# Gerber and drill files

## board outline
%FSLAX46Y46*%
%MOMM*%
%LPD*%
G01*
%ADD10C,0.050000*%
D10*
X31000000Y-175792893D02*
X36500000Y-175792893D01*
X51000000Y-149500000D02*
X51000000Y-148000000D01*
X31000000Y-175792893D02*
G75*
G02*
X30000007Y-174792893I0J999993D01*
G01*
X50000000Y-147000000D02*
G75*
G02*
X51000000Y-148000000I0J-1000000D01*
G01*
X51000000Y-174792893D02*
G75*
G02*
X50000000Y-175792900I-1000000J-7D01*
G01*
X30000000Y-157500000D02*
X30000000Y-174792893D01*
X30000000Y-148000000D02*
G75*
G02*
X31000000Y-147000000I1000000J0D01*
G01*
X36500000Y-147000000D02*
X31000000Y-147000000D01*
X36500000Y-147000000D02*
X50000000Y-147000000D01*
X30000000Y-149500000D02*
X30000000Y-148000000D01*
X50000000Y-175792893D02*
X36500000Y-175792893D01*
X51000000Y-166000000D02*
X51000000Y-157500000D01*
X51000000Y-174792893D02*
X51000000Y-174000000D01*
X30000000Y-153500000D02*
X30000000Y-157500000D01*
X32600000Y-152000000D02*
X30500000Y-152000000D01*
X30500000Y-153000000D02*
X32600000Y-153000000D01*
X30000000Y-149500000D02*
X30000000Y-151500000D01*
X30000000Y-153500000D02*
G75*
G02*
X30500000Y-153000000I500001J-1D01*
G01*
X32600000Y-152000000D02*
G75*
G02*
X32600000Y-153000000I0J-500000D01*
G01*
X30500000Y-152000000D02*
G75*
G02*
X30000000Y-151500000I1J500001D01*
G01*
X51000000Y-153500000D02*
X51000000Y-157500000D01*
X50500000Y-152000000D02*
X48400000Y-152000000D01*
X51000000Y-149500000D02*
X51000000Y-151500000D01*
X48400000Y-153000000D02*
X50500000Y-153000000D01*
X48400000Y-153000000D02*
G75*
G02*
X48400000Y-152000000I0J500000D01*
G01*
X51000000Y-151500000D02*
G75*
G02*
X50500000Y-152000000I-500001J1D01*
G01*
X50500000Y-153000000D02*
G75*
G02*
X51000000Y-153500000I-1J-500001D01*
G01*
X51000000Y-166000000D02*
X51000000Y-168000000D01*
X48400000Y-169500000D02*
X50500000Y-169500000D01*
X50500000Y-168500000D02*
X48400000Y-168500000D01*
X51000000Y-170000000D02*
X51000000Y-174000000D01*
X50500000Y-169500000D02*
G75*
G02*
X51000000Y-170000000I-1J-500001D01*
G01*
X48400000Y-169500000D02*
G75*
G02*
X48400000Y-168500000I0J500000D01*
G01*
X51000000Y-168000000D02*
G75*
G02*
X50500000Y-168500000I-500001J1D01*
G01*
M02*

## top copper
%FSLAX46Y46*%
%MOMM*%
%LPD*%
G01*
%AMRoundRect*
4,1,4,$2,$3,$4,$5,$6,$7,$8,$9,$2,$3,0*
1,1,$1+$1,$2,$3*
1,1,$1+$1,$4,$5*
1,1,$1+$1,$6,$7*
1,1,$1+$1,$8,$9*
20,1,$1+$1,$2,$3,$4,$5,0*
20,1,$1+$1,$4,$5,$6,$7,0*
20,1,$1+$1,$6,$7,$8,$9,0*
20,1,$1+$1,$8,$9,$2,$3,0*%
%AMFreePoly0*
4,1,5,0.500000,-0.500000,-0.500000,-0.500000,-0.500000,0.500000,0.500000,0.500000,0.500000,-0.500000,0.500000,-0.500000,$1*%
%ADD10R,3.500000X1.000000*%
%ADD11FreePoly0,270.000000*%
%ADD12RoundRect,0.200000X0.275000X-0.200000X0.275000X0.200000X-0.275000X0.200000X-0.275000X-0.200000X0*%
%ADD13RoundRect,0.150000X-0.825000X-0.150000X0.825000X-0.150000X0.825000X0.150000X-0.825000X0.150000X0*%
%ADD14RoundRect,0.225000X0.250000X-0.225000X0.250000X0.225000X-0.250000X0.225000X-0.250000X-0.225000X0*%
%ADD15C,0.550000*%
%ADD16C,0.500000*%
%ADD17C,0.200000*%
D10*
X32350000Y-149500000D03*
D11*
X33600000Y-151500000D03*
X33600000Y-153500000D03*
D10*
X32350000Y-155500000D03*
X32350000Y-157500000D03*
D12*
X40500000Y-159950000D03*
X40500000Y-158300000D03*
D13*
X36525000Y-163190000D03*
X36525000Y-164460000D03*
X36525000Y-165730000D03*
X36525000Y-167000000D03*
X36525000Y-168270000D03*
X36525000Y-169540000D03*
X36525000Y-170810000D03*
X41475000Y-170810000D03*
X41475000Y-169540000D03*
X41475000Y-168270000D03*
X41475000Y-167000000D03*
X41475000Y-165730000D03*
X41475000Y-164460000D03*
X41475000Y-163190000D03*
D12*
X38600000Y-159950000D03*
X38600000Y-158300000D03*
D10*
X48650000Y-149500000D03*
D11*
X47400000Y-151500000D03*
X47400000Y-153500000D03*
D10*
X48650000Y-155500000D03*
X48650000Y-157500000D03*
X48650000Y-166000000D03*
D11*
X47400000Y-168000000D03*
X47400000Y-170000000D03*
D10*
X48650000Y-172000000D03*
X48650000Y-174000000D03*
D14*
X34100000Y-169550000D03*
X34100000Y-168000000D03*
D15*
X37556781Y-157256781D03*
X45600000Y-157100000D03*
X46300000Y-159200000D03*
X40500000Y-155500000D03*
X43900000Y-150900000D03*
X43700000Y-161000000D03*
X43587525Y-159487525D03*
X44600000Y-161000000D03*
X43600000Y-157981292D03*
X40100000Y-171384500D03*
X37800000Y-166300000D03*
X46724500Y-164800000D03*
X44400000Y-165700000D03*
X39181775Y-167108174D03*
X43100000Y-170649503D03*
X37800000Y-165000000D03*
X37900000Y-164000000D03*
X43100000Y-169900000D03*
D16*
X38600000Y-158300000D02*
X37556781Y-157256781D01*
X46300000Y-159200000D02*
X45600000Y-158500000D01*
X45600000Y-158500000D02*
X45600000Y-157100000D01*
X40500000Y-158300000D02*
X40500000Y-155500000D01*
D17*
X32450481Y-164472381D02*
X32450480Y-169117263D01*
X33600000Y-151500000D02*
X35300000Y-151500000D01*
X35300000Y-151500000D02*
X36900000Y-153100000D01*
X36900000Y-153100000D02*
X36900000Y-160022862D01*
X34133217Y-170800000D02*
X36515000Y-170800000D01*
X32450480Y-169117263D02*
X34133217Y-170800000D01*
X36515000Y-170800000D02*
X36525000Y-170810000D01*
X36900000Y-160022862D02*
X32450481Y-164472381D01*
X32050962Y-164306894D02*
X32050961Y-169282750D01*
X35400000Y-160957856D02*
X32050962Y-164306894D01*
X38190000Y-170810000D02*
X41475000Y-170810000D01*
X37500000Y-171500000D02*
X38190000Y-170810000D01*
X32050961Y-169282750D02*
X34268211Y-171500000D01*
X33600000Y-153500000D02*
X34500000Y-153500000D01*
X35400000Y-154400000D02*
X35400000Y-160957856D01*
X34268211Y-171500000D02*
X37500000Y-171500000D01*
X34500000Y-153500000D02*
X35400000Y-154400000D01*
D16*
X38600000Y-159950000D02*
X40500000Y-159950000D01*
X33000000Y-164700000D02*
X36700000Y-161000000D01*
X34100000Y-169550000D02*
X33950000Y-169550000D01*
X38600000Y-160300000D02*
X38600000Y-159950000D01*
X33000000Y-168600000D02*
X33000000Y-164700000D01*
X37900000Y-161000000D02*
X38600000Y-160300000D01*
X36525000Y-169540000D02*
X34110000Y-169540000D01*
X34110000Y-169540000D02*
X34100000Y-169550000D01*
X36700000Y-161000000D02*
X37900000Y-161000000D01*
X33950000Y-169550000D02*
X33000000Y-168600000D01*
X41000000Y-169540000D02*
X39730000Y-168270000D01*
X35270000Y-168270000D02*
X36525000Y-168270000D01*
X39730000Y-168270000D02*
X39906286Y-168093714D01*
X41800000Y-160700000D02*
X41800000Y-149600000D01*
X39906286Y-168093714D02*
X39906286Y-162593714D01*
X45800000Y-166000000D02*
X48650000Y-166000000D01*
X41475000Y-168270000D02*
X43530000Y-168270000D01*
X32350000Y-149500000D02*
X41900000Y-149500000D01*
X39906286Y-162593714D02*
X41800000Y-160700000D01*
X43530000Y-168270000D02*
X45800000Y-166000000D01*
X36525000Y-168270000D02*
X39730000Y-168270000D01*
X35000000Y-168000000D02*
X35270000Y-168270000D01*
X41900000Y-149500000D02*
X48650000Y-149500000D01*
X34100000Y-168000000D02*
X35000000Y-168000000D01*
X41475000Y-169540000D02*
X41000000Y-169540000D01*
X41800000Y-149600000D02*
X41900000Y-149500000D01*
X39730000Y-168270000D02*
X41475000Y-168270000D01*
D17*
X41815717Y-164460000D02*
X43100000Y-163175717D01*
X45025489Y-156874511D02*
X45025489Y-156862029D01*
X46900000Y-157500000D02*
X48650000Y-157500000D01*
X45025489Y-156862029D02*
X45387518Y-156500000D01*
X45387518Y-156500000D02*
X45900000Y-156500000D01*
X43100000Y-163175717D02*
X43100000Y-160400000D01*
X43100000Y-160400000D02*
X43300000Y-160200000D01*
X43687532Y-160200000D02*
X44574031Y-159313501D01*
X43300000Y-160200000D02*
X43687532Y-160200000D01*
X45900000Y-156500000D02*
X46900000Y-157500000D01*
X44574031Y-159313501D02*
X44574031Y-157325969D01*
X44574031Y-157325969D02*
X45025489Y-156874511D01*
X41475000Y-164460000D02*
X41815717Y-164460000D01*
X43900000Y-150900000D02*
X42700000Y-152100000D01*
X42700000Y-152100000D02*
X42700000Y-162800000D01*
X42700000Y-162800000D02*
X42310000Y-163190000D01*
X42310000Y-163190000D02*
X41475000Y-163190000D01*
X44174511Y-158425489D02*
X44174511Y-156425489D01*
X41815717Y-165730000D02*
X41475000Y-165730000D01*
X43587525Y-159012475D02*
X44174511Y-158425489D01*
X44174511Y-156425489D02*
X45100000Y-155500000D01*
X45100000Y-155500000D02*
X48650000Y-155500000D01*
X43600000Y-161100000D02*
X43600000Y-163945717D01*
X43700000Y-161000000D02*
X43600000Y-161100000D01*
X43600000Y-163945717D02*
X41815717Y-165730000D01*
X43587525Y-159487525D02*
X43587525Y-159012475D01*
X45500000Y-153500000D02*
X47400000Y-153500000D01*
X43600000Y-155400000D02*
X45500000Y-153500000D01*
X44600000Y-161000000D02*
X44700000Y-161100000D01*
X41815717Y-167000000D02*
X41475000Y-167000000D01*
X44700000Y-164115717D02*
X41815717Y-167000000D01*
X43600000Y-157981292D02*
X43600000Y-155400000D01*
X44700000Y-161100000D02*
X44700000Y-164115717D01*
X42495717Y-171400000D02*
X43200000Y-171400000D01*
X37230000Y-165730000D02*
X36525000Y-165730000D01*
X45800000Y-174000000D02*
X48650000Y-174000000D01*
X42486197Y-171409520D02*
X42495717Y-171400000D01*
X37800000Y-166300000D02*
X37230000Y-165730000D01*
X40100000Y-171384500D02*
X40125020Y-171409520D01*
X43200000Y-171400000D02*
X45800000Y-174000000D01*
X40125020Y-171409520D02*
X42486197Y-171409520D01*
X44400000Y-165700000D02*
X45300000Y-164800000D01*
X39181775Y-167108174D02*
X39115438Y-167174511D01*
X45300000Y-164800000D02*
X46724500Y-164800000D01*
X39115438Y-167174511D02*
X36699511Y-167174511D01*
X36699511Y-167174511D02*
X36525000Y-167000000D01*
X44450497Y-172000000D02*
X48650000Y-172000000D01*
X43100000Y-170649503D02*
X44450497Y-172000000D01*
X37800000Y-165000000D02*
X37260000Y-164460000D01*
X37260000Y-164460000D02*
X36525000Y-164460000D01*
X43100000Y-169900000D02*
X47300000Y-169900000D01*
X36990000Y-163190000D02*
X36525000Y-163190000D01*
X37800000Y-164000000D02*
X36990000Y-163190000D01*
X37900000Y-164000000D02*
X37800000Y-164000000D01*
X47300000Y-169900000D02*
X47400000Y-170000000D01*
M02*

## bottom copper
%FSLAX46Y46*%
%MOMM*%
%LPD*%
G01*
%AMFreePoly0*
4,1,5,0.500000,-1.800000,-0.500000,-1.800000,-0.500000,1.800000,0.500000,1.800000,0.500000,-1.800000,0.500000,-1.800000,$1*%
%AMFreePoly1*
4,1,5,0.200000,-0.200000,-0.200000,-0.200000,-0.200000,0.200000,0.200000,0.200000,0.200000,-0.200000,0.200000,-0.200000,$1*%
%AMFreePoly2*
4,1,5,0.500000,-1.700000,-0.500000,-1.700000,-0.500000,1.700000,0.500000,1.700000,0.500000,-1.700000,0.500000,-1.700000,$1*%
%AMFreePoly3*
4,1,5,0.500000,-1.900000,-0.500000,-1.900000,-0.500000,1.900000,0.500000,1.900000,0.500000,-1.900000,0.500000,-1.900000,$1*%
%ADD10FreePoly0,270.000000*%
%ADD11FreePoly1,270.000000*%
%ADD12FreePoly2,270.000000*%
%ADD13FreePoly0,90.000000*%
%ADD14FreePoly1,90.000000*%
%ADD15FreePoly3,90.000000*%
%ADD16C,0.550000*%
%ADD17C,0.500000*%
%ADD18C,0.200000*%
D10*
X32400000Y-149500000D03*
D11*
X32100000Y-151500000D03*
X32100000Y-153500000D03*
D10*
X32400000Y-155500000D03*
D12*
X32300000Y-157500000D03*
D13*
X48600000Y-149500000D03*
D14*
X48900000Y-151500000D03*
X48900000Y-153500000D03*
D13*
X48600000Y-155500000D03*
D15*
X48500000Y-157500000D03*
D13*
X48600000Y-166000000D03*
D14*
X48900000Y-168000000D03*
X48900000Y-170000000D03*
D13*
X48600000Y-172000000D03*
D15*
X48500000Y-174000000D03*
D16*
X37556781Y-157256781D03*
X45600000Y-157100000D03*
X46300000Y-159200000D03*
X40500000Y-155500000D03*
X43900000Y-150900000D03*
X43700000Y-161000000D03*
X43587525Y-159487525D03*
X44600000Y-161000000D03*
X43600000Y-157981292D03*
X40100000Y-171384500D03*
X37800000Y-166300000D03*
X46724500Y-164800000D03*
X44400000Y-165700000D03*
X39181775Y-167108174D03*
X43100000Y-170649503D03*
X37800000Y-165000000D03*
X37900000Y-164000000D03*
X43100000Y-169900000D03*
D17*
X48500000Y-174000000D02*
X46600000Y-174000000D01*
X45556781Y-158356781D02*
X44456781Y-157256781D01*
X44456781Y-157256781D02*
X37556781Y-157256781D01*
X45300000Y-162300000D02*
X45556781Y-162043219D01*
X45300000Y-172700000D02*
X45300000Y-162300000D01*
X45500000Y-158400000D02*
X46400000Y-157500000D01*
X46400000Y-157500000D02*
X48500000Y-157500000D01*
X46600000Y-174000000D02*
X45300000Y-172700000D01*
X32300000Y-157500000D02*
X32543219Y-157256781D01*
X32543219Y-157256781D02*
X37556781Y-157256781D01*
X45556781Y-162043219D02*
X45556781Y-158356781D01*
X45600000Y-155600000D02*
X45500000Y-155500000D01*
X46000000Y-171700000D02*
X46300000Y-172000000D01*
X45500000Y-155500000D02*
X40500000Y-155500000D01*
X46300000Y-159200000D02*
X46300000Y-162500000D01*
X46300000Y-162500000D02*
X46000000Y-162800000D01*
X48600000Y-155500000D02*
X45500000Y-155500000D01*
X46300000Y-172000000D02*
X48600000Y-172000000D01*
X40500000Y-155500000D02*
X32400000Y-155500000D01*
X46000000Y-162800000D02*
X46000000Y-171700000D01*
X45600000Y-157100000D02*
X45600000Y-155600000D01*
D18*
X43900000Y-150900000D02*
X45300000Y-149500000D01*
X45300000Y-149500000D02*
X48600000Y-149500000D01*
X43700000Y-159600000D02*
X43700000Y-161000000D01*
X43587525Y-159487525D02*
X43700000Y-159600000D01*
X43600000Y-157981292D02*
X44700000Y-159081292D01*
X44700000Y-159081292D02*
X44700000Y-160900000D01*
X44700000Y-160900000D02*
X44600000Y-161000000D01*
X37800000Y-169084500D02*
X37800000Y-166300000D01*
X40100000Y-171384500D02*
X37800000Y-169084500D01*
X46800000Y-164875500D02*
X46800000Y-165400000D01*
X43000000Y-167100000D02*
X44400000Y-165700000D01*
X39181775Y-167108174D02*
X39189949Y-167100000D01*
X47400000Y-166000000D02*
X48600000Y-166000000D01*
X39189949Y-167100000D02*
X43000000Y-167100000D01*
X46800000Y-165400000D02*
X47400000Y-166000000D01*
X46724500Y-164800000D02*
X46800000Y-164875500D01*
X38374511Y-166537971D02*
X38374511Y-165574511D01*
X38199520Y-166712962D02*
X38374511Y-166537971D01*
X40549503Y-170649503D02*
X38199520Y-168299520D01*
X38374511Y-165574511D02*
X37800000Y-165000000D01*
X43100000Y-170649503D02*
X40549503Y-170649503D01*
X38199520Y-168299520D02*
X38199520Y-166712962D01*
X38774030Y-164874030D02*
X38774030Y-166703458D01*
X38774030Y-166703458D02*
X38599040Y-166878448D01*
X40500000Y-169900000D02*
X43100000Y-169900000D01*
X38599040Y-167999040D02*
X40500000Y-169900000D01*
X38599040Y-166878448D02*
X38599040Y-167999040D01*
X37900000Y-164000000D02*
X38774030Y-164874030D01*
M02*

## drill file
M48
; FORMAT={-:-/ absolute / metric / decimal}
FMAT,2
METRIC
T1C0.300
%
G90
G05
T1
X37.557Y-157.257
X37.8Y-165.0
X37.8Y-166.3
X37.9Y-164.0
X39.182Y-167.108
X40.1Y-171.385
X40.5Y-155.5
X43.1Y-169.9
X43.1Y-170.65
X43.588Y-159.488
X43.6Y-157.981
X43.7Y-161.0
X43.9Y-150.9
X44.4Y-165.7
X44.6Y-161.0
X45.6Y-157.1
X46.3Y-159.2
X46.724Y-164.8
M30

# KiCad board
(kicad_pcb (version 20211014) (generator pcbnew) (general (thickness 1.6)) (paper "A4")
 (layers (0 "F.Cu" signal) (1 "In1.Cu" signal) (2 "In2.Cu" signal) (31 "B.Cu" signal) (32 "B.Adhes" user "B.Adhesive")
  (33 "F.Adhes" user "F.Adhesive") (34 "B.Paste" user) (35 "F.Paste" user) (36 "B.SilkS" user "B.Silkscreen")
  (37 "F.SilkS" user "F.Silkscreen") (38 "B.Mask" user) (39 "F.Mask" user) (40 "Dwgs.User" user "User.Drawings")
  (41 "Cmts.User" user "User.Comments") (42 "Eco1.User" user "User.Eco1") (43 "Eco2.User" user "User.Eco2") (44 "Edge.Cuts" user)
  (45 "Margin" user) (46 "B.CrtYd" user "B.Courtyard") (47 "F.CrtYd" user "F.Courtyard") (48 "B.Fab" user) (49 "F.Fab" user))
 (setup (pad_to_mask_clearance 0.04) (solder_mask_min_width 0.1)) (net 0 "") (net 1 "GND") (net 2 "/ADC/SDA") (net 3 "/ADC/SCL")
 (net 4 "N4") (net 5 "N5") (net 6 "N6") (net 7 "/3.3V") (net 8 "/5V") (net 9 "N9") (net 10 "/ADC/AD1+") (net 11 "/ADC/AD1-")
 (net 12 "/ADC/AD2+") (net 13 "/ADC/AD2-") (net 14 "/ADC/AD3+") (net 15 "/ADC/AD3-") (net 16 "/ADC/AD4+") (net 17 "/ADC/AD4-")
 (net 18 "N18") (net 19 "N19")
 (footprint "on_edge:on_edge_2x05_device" (layer "F.Cu") (at 30 153.5 -90)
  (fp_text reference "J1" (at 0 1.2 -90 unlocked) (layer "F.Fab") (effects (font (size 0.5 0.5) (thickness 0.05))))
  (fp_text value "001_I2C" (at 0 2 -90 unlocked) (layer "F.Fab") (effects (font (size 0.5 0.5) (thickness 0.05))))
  (fp_line (start 0 0) (end 4 0) (layer "Edge.Cuts") (width 0.05))
  (fp_line (start -1.5 -2.6) (end -1.5 -0.5) (layer "Edge.Cuts") (width 0.05))
  (fp_line (start -0.5 -0.5) (end -0.5 -2.6) (layer "Edge.Cuts") (width 0.05))
  (fp_line (start -4 0) (end -2 0) (layer "Edge.Cuts") (width 0.05))
  (fp_arc (start 0 0) (mid -0.353553 -0.146447) (end -0.5 -0.5) (layer "Edge.Cuts") (width 0.05))
  (fp_arc (start -1.5 -2.6) (mid -1 -3.1) (end -0.5 -2.6) (layer "Edge.Cuts") (width 0.05))
  (fp_arc (start -1.5 -0.5) (mid -1.646447 -0.146447) (end -2 0) (layer "Edge.Cuts") (width 0.05))
  (pad "1" smd rect locked (at -4 -2.35 90) (size 1 3.5) (layers "F.Cu" "F.Mask") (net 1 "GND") (zone_connect 0))
  (pad "2" smd custom locked (at -2 -3.6 270) (size 1 1) (layers "F.Cu" "F.Mask") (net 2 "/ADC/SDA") (zone_connect 0)
   (options (clearance outline) (anchor rect)) (primitives))
  (pad "3" smd custom locked (at 0 -3.6 270) (size 1 1) (layers "F.Cu" "F.Mask") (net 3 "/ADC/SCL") (zone_connect 0)
   (options (clearance outline) (anchor rect)) (primitives))
  (pad "4" smd rect locked (at 2 -2.35 90) (size 1 3.5) (layers "F.Cu" "F.Mask") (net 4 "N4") (zone_connect 0))
  (pad "5" smd rect locked (at 4 -2.35 90) (size 1 3.5) (layers "F.Cu" "F.Mask") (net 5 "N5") (zone_connect 0))
  (pad "6" smd custom locked (at -4 -2.4 270) (size 1 3.6) (layers "B.Cu" "B.Mask") (zone_connect 0)
   (options (clearance outline) (anchor rect)) (primitives))
  (pad "7" smd custom locked (at -2 -2.1 270) (size 0.4 0.4) (layers "B.Cu" "B.Mask") (zone_connect 0)
   (options (clearance outline) (anchor rect)) (primitives))
  (pad "8" smd custom locked (at 0 -2.1 270) (size 0.4 0.4) (layers "B.Cu" "B.Mask") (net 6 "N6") (zone_connect 0)
   (options (clearance outline) (anchor rect)) (primitives))
  (pad "9" smd custom locked (at 2 -2.4 270) (size 1 3.6) (layers "B.Cu" "B.Mask") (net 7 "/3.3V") (zone_connect 0)
   (options (clearance outline) (anchor rect)) (primitives))
  (pad "10" smd custom locked (at 4 -2.3 270) (size 1 3.4) (layers "B.Cu" "B.Mask") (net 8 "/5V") (zone_connect 0)
   (options (clearance outline) (anchor rect)) (primitives)))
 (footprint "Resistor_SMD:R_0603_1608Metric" (layer "F.Cu") (at 40.5 159.125 90)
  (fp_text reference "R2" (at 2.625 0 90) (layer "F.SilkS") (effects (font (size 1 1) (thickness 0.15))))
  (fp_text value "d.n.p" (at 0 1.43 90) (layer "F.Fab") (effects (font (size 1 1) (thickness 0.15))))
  (pad "1" smd roundrect locked (at -0.825 0 90) (size 0.8 0.95) (layers "F.Cu" "F.Paste" "F.Mask") (roundrect_rratio 0.25) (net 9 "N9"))
  (pad "2" smd roundrect locked (at 0.825 0 90) (size 0.8 0.95) (layers "F.Cu" "F.Paste" "F.Mask") (roundrect_rratio 0.25) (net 7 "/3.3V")))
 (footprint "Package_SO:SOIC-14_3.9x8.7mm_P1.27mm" (layer "F.Cu") (at 39 167)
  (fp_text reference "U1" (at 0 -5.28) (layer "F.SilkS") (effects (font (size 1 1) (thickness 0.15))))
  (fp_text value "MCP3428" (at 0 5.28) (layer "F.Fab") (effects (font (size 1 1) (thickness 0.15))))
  (pad "1" smd roundrect locked (at -2.475 -3.81) (size 1.95 0.6) (layers "F.Cu" "F.Paste" "F.Mask") (roundrect_rratio 0.25)
   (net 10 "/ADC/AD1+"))
  (pad "2" smd roundrect locked (at -2.475 -2.54) (size 1.95 0.6) (layers "F.Cu" "F.Paste" "F.Mask") (roundrect_rratio 0.25)
   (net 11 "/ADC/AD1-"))
  (pad "3" smd roundrect locked (at -2.475 -1.27) (size 1.95 0.6) (layers "F.Cu" "F.Paste" "F.Mask") (roundrect_rratio 0.25)
   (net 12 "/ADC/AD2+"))
  (pad "4" smd roundrect locked (at -2.475 0) (size 1.95 0.6) (layers "F.Cu" "F.Paste" "F.Mask") (roundrect_rratio 0.25)
   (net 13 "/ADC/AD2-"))
  (pad "5" smd roundrect locked (at -2.475 1.27) (size 1.95 0.6) (layers "F.Cu" "F.Paste" "F.Mask") (roundrect_rratio 0.25) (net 1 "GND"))
  (pad "6" smd roundrect locked (at -2.475 2.54) (size 1.95 0.6) (layers "F.Cu" "F.Paste" "F.Mask") (roundrect_rratio 0.25) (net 9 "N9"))
  (pad "7" smd roundrect locked (at -2.475 3.81) (size 1.95 0.6) (layers "F.Cu" "F.Paste" "F.Mask") (roundrect_rratio 0.25)
   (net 2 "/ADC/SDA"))
  (pad "8" smd roundrect locked (at 2.475 3.81) (size 1.95 0.6) (layers "F.Cu" "F.Paste" "F.Mask") (roundrect_rratio 0.25)
   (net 3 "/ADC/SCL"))
  (pad "9" smd roundrect locked (at 2.475 2.54) (size 1.95 0.6) (layers "F.Cu" "F.Paste" "F.Mask") (roundrect_rratio 0.25) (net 1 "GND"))
  (pad "10" smd roundrect locked (at 2.475 1.27) (size 1.95 0.6) (layers "F.Cu" "F.Paste" "F.Mask") (roundrect_rratio 0.25) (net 1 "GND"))
  (pad "11" smd roundrect locked (at 2.475 0) (size 1.95 0.6) (layers "F.Cu" "F.Paste" "F.Mask") (roundrect_rratio 0.25)
   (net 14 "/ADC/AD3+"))
  (pad "12" smd roundrect locked (at 2.475 -1.27) (size 1.95 0.6) (layers "F.Cu" "F.Paste" "F.Mask") (roundrect_rratio 0.25)
   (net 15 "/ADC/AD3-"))
  (pad "13" smd roundrect locked (at 2.475 -2.54) (size 1.95 0.6) (layers "F.Cu" "F.Paste" "F.Mask") (roundrect_rratio 0.25)
   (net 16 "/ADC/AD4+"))
  (pad "14" smd roundrect locked (at 2.475 -3.81) (size 1.95 0.6) (layers "F.Cu" "F.Paste" "F.Mask") (roundrect_rratio 0.25)
   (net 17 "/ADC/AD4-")))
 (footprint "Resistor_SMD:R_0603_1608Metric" (layer "F.Cu") (at 38.6 159.125 90)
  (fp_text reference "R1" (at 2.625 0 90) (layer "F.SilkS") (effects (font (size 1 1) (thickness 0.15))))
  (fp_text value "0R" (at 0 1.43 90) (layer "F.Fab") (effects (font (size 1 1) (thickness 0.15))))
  (pad "1" smd roundrect locked (at -0.825 0 90) (size 0.8 0.95) (layers "F.Cu" "F.Paste" "F.Mask") (roundrect_rratio 0.25) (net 9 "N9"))
  (pad "2" smd roundrect locked (at 0.825 0 90) (size 0.8 0.95) (layers "F.Cu" "F.Paste" "F.Mask") (roundrect_rratio 0.25) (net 8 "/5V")))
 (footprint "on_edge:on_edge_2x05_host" (layer "F.Cu") (at 51 153.5 -90)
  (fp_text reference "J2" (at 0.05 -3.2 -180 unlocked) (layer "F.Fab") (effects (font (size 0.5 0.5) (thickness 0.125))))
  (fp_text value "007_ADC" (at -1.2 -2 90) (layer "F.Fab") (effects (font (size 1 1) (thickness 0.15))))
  (fp_line (start 0 0) (end 4 0) (layer "Edge.Cuts") (width 0.05))
  (fp_line (start -1.5 0.5) (end -1.5 2.6) (layer "Edge.Cuts") (width 0.05))
  (fp_line (start -4 0) (end -2 0) (layer "Edge.Cuts") (width 0.05))
  (fp_line (start -0.5 2.6) (end -0.5 0.5) (layer "Edge.Cuts") (width 0.05))
  (fp_arc (start -0.5 2.6) (mid -1 3.1) (end -1.5 2.6) (layer "Edge.Cuts") (width 0.05))
  (fp_arc (start -2 0) (mid -1.646447 0.146447) (end -1.5 0.5) (layer "Edge.Cuts") (width 0.05))
  (fp_arc (start -0.5 0.5) (mid -0.353553 0.146447) (end 0 0) (layer "Edge.Cuts") (width 0.05))
  (pad "1" smd rect locked (at -4 2.35 270) (size 1 3.5) (layers "F.Cu" "F.Mask") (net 1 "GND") (zone_connect 0))
  (pad "2" smd custom locked (at -2 3.6 270) (size 1 1) (layers "F.Cu" "F.Mask") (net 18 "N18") (zone_connect 0)
   (options (clearance outline) (anchor rect)) (primitives))
  (pad "3" smd custom locked (at 0 3.6 270) (size 1 1) (layers "F.Cu" "F.Mask") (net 14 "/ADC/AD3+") (zone_connect 0)
   (options (clearance outline) (anchor rect)) (primitives))
  (pad "4" smd rect locked (at 2 2.35 270) (size 1 3.5) (layers "F.Cu" "F.Mask") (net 15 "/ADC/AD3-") (zone_connect 0))
  (pad "5" smd rect locked (at 4 2.35 270) (size 1 3.5) (layers "F.Cu" "F.Mask") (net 16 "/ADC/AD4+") (zone_connect 0))
  (pad "6" smd custom locked (at -4 2.4 90) (size 1 3.6) (layers "B.Cu" "B.Mask") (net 17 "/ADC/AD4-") (zone_connect 0)
   (options (clearance outline) (anchor rect)) (primitives))
  (pad "7" smd custom locked (at -2 2.1 90) (size 0.4 0.4) (layers "B.Cu" "B.Mask") (zone_connect 0)
   (options (clearance outline) (anchor rect)) (primitives))
  (pad "8" smd custom locked (at 0 2.1 90) (size 0.4 0.4) (layers "B.Cu" "B.Mask") (zone_connect 0)
   (options (clearance outline) (anchor rect)) (primitives))
  (pad "9" smd custom locked (at 2 2.4 90) (size 1 3.6) (layers "B.Cu" "B.Mask") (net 7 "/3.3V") (zone_connect 0)
   (options (clearance outline) (anchor rect)) (primitives))
  (pad "10" smd custom locked (at 4 2.5 90) (size 1 3.8) (layers "B.Cu" "B.Mask") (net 8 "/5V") (zone_connect 0)
   (options (clearance outline) (anchor rect)) (primitives)))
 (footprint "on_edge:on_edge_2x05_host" (layer "F.Cu") (at 51 170 -90)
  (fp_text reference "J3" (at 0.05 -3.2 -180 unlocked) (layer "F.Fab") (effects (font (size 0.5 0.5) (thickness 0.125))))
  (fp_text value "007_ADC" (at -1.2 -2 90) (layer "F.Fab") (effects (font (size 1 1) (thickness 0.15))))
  (fp_line (start -4 0) (end -2 0) (layer "Edge.Cuts") (width 0.05))
  (fp_line (start -0.5 2.6) (end -0.5 0.5) (layer "Edge.Cuts") (width 0.05))
  (fp_line (start -1.5 0.5) (end -1.5 2.6) (layer "Edge.Cuts") (width 0.05))
  (fp_line (start 0 0) (end 4 0) (layer "Edge.Cuts") (width 0.05))
  (fp_arc (start -0.5 0.5) (mid -0.353553 0.146447) (end 0 0) (layer "Edge.Cuts") (width 0.05))
  (fp_arc (start -0.5 2.6) (mid -1 3.1) (end -1.5 2.6) (layer "Edge.Cuts") (width 0.05))
  (fp_arc (start -2 0) (mid -1.646447 0.146447) (end -1.5 0.5) (layer "Edge.Cuts") (width 0.05))
  (pad "1" smd rect locked (at -4 2.35 270) (size 1 3.5) (layers "F.Cu" "F.Mask") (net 1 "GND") (zone_connect 0))
  (pad "2" smd custom locked (at -2 3.6 270) (size 1 1) (layers "F.Cu" "F.Mask") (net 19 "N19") (zone_connect 0)
   (options (clearance outline) (anchor rect)) (primitives))
  (pad "3" smd custom locked (at 0 3.6 270) (size 1 1) (layers "F.Cu" "F.Mask") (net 10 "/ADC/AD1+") (zone_connect 0)
   (options (clearance outline) (anchor rect)) (primitives))
  (pad "4" smd rect locked (at 2 2.35 270) (size 1 3.5) (layers "F.Cu" "F.Mask") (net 11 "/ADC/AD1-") (zone_connect 0))
  (pad "5" smd rect locked (at 4 2.35 270) (size 1 3.5) (layers "F.Cu" "F.Mask") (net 12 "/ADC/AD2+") (zone_connect 0))
  (pad "6" smd custom locked (at -4 2.4 90) (size 1 3.6) (layers "B.Cu" "B.Mask") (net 13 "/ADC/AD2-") (zone_connect 0)
   (options (clearance outline) (anchor rect)) (primitives))
  (pad "7" smd custom locked (at -2 2.1 90) (size 0.4 0.4) (layers "B.Cu" "B.Mask") (zone_connect 0)
   (options (clearance outline) (anchor rect)) (primitives))
  (pad "8" smd custom locked (at 0 2.1 90) (size 0.4 0.4) (layers "B.Cu" "B.Mask") (zone_connect 0)
   (options (clearance outline) (anchor rect)) (primitives))
  (pad "9" smd custom locked (at 2 2.4 90) (size 1 3.6) (layers "B.Cu" "B.Mask") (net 7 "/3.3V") (zone_connect 0)
   (options (clearance outline) (anchor rect)) (primitives))
  (pad "10" smd custom locked (at 4 2.5 90) (size 1 3.8) (layers "B.Cu" "B.Mask") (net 8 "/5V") (zone_connect 0)
   (options (clearance outline) (anchor rect)) (primitives)))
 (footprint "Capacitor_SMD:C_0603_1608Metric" (layer "F.Cu") (at 34.1 168.775 90)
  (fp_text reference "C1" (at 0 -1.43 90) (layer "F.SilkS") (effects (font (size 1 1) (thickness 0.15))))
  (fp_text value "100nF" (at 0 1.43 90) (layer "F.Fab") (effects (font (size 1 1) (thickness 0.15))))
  (pad "1" smd roundrect locked (at -0.775 0 90) (size 0.9 0.95) (layers "F.Cu" "F.Paste" "F.Mask") (roundrect_rratio 0.25) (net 9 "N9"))
  (pad "2" smd roundrect locked (at 0.775 0 90) (size 0.9 0.95) (layers "F.Cu" "F.Paste" "F.Mask") (roundrect_rratio 0.25) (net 1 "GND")))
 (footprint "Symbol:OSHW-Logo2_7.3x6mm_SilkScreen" (layer "B.Cu") (at 40.4 172.892893 180)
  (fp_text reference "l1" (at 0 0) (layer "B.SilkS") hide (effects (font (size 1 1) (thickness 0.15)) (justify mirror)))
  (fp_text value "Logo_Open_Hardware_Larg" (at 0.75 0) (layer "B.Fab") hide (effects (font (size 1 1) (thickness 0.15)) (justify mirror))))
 (gr_line (start 31 175.792893) (end 36.5 175.792893) (layer "Edge.Cuts") (width 0.05))
 (gr_line (start 51 149.5) (end 51 148) (layer "Edge.Cuts") (width 0.05))
 (gr_arc (start 31 175.792893) (mid 30.292893 175.5) (end 30 174.792893) (layer "Edge.Cuts") (width 0.05))
 (gr_arc (start 50 147) (mid 50.707107 147.292893) (end 51 148) (layer "Edge.Cuts") (width 0.05))
 (gr_arc (start 51 174.792893) (mid 50.707107 175.5) (end 50 175.792893) (layer "Edge.Cuts") (width 0.05))
 (gr_line (start 30 157.5) (end 30 174.792893) (layer "Edge.Cuts") (width 0.05))
 (gr_arc (start 30 148) (mid 30.292893 147.292893) (end 31 147) (layer "Edge.Cuts") (width 0.05))
 (gr_line (start 36.5 147) (end 31 147) (layer "Edge.Cuts") (width 0.05))
 (gr_line (start 36.5 147) (end 50 147) (layer "Edge.Cuts") (width 0.05))
 (gr_line (start 30 149.5) (end 30 148) (layer "Edge.Cuts") (width 0.05))
 (gr_line (start 50 175.792893) (end 36.5 175.792893) (layer "Edge.Cuts") (width 0.05))
 (gr_line (start 51 166) (end 51 157.5) (layer "Edge.Cuts") (width 0.05))
 (gr_line (start 51 174.792893) (end 51 174) (layer "Edge.Cuts") (width 0.05))
 (segment (start 38.6 158.3) (end 37.556781 157.256781) (width 0.5) (layer "F.Cu") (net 8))
 (via (at 37.556781 157.256781) (size 0.55) (drill 0.3) (layers "F.Cu" "B.Cu") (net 8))
 (segment (start 48.5 174) (end 46.6 174) (width 0.5) (layer "B.Cu") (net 8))
 (segment (start 45.556781 158.356781) (end 44.456781 157.256781) (width 0.5) (layer "B.Cu") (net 8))
 (segment (start 44.456781 157.256781) (end 37.556781 157.256781) (width 0.5) (layer "B.Cu") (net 8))
 (segment (start 45.3 162.3) (end 45.556781 162.043219) (width 0.5) (layer "B.Cu") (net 8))
 (segment (start 45.3 172.7) (end 45.3 162.3) (width 0.5) (layer "B.Cu") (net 8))
 (segment (start 45.5 158.4) (end 46.4 157.5) (width 0.5) (layer "B.Cu") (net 8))
 (segment (start 46.4 157.5) (end 48.5 157.5) (width 0.5) (layer "B.Cu") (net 8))
 (segment (start 46.6 174) (end 45.3 172.7) (width 0.5) (layer "B.Cu") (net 8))
 (segment (start 32.3 157.5) (end 32.543219 157.256781) (width 0.5) (layer "B.Cu") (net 8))
 (segment (start 32.543219 157.256781) (end 37.556781 157.256781) (width 0.5) (layer "B.Cu") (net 8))
 (segment (start 45.556781 162.043219) (end 45.556781 158.356781) (width 0.5) (layer "B.Cu") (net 8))
 (segment (start 46.3 159.2) (end 45.6 158.5) (width 0.5) (layer "F.Cu") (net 7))
 (segment (start 45.6 158.5) (end 45.6 157.1) (width 0.5) (layer "F.Cu") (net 7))
 (segment (start 40.5 158.3) (end 40.5 155.5) (width 0.5) (layer "F.Cu") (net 7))
 (via (at 45.6 157.1) (size 0.55) (drill 0.3) (layers "F.Cu" "B.Cu") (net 7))
 (via (at 46.3 159.2) (size 0.55) (drill 0.3) (layers "F.Cu" "B.Cu") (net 7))
 (via (at 40.5 155.5) (size 0.55) (drill 0.3) (layers "F.Cu" "B.Cu") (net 7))
 (segment (start 45.6 155.6) (end 45.5 155.5) (width 0.5) (layer "B.Cu") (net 7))
 (segment (start 46 171.7) (end 46.3 172) (width 0.5) (layer "B.Cu") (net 7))
 (segment (start 45.5 155.5) (end 40.5 155.5) (width 0.5) (layer "B.Cu") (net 7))
 (segment (start 46.3 159.2) (end 46.3 162.5) (width 0.5) (layer "B.Cu") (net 7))
 (segment (start 46.3 162.5) (end 46 162.8) (width 0.5) (layer "B.Cu") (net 7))
 (segment (start 48.6 155.5) (end 45.5 155.5) (width 0.5) (layer "B.Cu") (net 7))
 (segment (start 46.3 172) (end 48.6 172) (width 0.5) (layer "B.Cu") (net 7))
 (segment (start 40.5 155.5) (end 32.4 155.5) (width 0.5) (layer "B.Cu") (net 7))
 (segment (start 46 162.8) (end 46 171.7) (width 0.5) (layer "B.Cu") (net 7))
 (segment (start 45.6 157.1) (end 45.6 155.6) (width 0.5) (layer "B.Cu") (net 7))
 (segment (start 32.450481 164.472381) (end 32.45048 169.117263) (width 0.2) (layer "F.Cu") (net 2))
 (segment (start 33.6 151.5) (end 35.3 151.5) (width 0.2) (layer "F.Cu") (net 2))
 (segment (start 35.3 151.5) (end 36.9 153.1) (width 0.2) (layer "F.Cu") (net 2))
 (segment (start 36.9 153.1) (end 36.9 160.022862) (width 0.2) (layer "F.Cu") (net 2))
 (segment (start 34.133217 170.8) (end 36.515 170.8) (width 0.2) (layer "F.Cu") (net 2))
 (segment (start 32.45048 169.117263) (end 34.133217 170.8) (width 0.2) (layer "F.Cu") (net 2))
 (segment (start 36.515 170.8) (end 36.525 170.81) (width 0.2) (layer "F.Cu") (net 2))
 (segment (start 36.9 160.022862) (end 32.450481 164.472381) (width 0.2) (layer "F.Cu") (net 2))
 (segment (start 32.050962 164.306894) (end 32.050961 169.28275) (width 0.2) (layer "F.Cu") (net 3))
 (segment (start 35.4 160.957856) (end 32.050962 164.306894) (width 0.2) (layer "F.Cu") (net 3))
 (segment (start 38.19 170.81) (end 41.475 170.81) (width 0.2) (layer "F.Cu") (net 3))
 (segment (start 37.5 171.5) (end 38.19 170.81) (width 0.2) (layer "F.Cu") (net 3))
 (segment (start 32.050961 169.28275) (end 34.268211 171.5) (width 0.2) (layer "F.Cu") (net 3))
 (segment (start 33.6 153.5) (end 34.5 153.5) (width 0.2) (layer "F.Cu") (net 3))
 (segment (start 35.4 154.4) (end 35.4 160.957856) (width 0.2) (layer "F.Cu") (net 3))
 (segment (start 34.268211 171.5) (end 37.5 171.5) (width 0.2) (layer "F.Cu") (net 3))
 (segment (start 34.5 153.5) (end 35.4 154.4) (width 0.2) (layer "F.Cu") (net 3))
 (segment (start 38.6 159.95) (end 40.5 159.95) (width 0.5) (layer "F.Cu") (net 9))
 (segment (start 33 164.7) (end 36.7 161) (width 0.5) (layer "F.Cu") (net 9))
 (segment (start 34.1 169.55) (end 33.95 169.55) (width 0.5) (layer "F.Cu") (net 9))
 (segment (start 38.6 160.3) (end 38.6 159.95) (width 0.5) (layer "F.Cu") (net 9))
 (segment (start 33 168.6) (end 33 164.7) (width 0.5) (layer "F.Cu") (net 9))
 (segment (start 37.9 161) (end 38.6 160.3) (width 0.5) (layer "F.Cu") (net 9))
 (segment (start 36.525 169.54) (end 34.11 169.54) (width 0.5) (layer "F.Cu") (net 9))
 (segment (start 34.11 169.54) (end 34.1 169.55) (width 0.5) (layer "F.Cu") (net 9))
 (segment (start 36.7 161) (end 37.9 161) (width 0.5) (layer "F.Cu") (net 9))
 (segment (start 33.95 169.55) (end 33 168.6) (width 0.5) (layer "F.Cu") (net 9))
 (segment (start 41 169.54) (end 39.73 168.27) (width 0.5) (layer "F.Cu") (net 1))
 (segment (start 35.27 168.27) (end 36.525 168.27) (width 0.5) (layer "F.Cu") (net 1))
 (segment (start 39.73 168.27) (end 39.906286 168.093714) (width 0.5) (layer "F.Cu") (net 1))
 (segment (start 41.8 160.7) (end 41.8 149.6) (width 0.5) (layer "F.Cu") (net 1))
 (segment (start 39.906286 168.093714) (end 39.906286 162.593714) (width 0.5) (layer "F.Cu") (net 1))
 (segment (start 45.8 166) (end 48.65 166) (width 0.5) (layer "F.Cu") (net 1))
 (segment (start 41.475 168.27) (end 43.53 168.27) (width 0.5) (layer "F.Cu") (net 1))
 (segment (start 32.35 149.5) (end 41.9 149.5) (width 0.5) (layer "F.Cu") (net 1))
 (segment (start 39.906286 162.593714) (end 41.8 160.7) (width 0.5) (layer "F.Cu") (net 1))
 (segment (start 43.53 168.27) (end 45.8 166) (width 0.5) (layer "F.Cu") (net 1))
 (segment (start 36.525 168.27) (end 39.73 168.27) (width 0.5) (layer "F.Cu") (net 1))
 (segment (start 35 168) (end 35.27 168.27) (width 0.5) (layer "F.Cu") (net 1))
 (segment (start 41.9 149.5) (end 48.65 149.5) (width 0.5) (layer "F.Cu") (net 1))
 (segment (start 34.1 168) (end 35 168) (width 0.5) (layer "F.Cu") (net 1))
 (segment (start 41.475 169.54) (end 41 169.54) (width 0.5) (layer "F.Cu") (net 1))
 (segment (start 41.8 149.6) (end 41.9 149.5) (width 0.5) (layer "F.Cu") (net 1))
 (segment (start 39.73 168.27) (end 41.475 168.27) (width 0.5) (layer "F.Cu") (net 1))
 (segment (start 41.815717 164.46) (end 43.1 163.175717) (width 0.2) (layer "F.Cu") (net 16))
 (segment (start 45.025489 156.874511) (end 45.025489 156.862029) (width 0.2) (layer "F.Cu") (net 16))
 (segment (start 46.9 157.5) (end 48.65 157.5) (width 0.2) (layer "F.Cu") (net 16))
 (segment (start 45.025489 156.862029) (end 45.387518 156.5) (width 0.2) (layer "F.Cu") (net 16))
 (segment (start 45.387518 156.5) (end 45.9 156.5) (width 0.2) (layer "F.Cu") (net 16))
 (segment (start 43.1 163.175717) (end 43.1 160.4) (width 0.2) (layer "F.Cu") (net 16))
 (segment (start 43.1 160.4) (end 43.3 160.2) (width 0.2) (layer "F.Cu") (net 16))
 (segment (start 43.687532 160.2) (end 44.574031 159.313501) (width 0.2) (layer "F.Cu") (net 16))
 (segment (start 43.3 160.2) (end 43.687532 160.2) (width 0.2) (layer "F.Cu") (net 16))
 (segment (start 45.9 156.5) (end 46.9 157.5) (width 0.2) (layer "F.Cu") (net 16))
 (segment (start 44.574031 159.313501) (end 44.574031 157.325969) (width 0.2) (layer "F.Cu") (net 16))
 (segment (start 44.574031 157.325969) (end 45.025489 156.874511) (width 0.2) (layer "F.Cu") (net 16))
 (segment (start 41.475 164.46) (end 41.815717 164.46) (width 0.2) (layer "F.Cu") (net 16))
 (segment (start 43.9 150.9) (end 42.7 152.1) (width 0.2) (layer "F.Cu") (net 17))
 (segment (start 42.7 152.1) (end 42.7 162.8) (width 0.2) (layer "F.Cu") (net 17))
 (segment (start 42.7 162.8) (end 42.31 163.19) (width 0.2) (layer "F.Cu") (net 17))
 (segment (start 42.31 163.19) (end 41.475 163.19) (width 0.2) (layer "F.Cu") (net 17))
 (via (at 43.9 150.9) (size 0.55) (drill 0.3) (layers "F.Cu" "B.Cu") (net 17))
 (segment (start 43.9 150.9) (end 45.3 149.5) (width 0.2) (layer "B.Cu") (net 17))
 (segment (start 45.3 149.5) (end 48.6 149.5) (width 0.2) (layer "B.Cu") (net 17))
 (segment (start 44.174511 158.425489) (end 44.174511 156.425489) (width 0.2) (layer "F.Cu") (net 15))
 (segment (start 41.815717 165.73) (end 41.475 165.73) (width 0.2) (layer "F.Cu") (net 15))
 (segment (start 43.587525 159.012475) (end 44.174511 158.425489) (width 0.2) (layer "F.Cu") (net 15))
 (segment (start 44.174511 156.425489) (end 45.1 155.5) (width 0.2) (layer "F.Cu") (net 15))
 (segment (start 45.1 155.5) (end 48.65 155.5) (width 0.2) (layer "F.Cu") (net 15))
 (segment (start 43.6 161.1) (end 43.6 163.945717) (width 0.2) (layer "F.Cu") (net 15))
 (segment (start 43.7 161) (end 43.6 161.1) (width 0.2) (layer "F.Cu") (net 15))
 (segment (start 43.6 163.945717) (end 41.815717 165.73) (width 0.2) (layer "F.Cu") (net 15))
 (segment (start 43.587525 159.487525) (end 43.587525 159.012475) (width 0.2) (layer "F.Cu") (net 15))
 (via (at 43.7 161) (size 0.55) (drill 0.3) (layers "F.Cu" "B.Cu") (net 15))
 (via (at 43.587525 159.487525) (size 0.55) (drill 0.3) (layers "F.Cu" "B.Cu") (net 15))
 (segment (start 43.7 159.6) (end 43.7 161) (width 0.2) (layer "B.Cu") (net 15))
 (segment (start 43.587525 159.487525) (end 43.7 159.6) (width 0.2) (layer "B.Cu") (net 15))
 (segment (start 45.5 153.5) (end 47.4 153.5) (width 0.2) (layer "F.Cu") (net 14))
 (segment (start 43.6 155.4) (end 45.5 153.5) (width 0.2) (layer "F.Cu") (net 14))
 (segment (start 44.6 161) (end 44.7 161.1) (width 0.2) (layer "F.Cu") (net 14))
 (segment (start 41.815717 167) (end 41.475 167) (width 0.2) (layer "F.Cu") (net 14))
 (segment (start 44.7 164.115717) (end 41.815717 167) (width 0.2) (layer "F.Cu") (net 14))
 (segment (start 43.6 157.981292) (end 43.6 155.4) (width 0.2) (layer "F.Cu") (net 14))
 (segment (start 44.7 161.1) (end 44.7 164.115717) (width 0.2) (layer "F.Cu") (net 14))
 (via (at 44.6 161) (size 0.55) (drill 0.3) (layers "F.Cu" "B.Cu") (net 14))
 (via (at 43.6 157.981292) (size 0.55) (drill 0.3) (layers "F.Cu" "B.Cu") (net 14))
 (segment (start 43.6 157.981292) (end 44.7 159.081292) (width 0.2) (layer "B.Cu") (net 14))
 (segment (start 44.7 159.081292) (end 44.7 160.9) (width 0.2) (layer "B.Cu") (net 14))
 (segment (start 44.7 160.9) (end 44.6 161) (width 0.2) (layer "B.Cu") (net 14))
 (segment (start 42.495717 171.4) (end 43.2 171.4) (width 0.2) (layer "F.Cu") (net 12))
 (segment (start 37.23 165.73) (end 36.525 165.73) (width 0.2) (layer "F.Cu") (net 12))
 (segment (start 45.8 174) (end 48.65 174) (width 0.2) (layer "F.Cu") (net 12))
 (segment (start 42.486197 171.40952) (end 42.495717 171.4) (width 0.2) (layer "F.Cu") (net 12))
 (segment (start 37.8 166.3) (end 37.23 165.73) (width 0.2) (layer "F.Cu") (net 12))
 (segment (start 40.1 171.3845) (end 40.12502 171.40952) (width 0.2) (layer "F.Cu") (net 12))
 (segment (start 43.2 171.4) (end 45.8 174) (width 0.2) (layer "F.Cu") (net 12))
 (segment (start 40.12502 171.40952) (end 42.486197 171.40952) (width 0.2) (layer "F.Cu") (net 12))
 (via (at 40.1 171.3845) (size 0.55) (drill 0.3) (layers "F.Cu" "B.Cu") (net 12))
 (via (at 37.8 166.3) (size 0.55) (drill 0.3) (layers "F.Cu" "B.Cu") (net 12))
 (segment (start 37.8 169.0845) (end 37.8 166.3) (width 0.2) (layer "B.Cu") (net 12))
 (segment (start 40.1 171.3845) (end 37.8 169.0845) (width 0.2) (layer "B.Cu") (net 12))
 (segment (start 44.4 165.7) (end 45.3 164.8) (width 0.2) (layer "F.Cu") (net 13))
 (segment (start 39.181775 167.108174) (end 39.115438 167.174511) (width 0.2) (layer "F.Cu") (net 13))
 (segment (start 45.3 164.8) (end 46.7245 164.8) (width 0.2) (layer "F.Cu") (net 13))
 (segment (start 39.115438 167.174511) (end 36.699511 167.174511) (width 0.2) (layer "F.Cu") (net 13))
 (segment (start 36.699511 167.174511) (end 36.525 167) (width 0.2) (layer "F.Cu") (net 13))
 (via (at 46.7245 164.8) (size 0.55) (drill 0.3) (layers "F.Cu" "B.Cu") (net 13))
 (via (at 44.4 165.7) (size 0.55) (drill 0.3) (layers "F.Cu" "B.Cu") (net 13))
 (via (at 39.181775 167.108174) (size 0.55) (drill 0.3) (layers "F.Cu" "B.Cu") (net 13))
 (segment (start 46.8 164.8755) (end 46.8 165.4) (width 0.2) (layer "B.Cu") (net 13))
 (segment (start 43 167.1) (end 44.4 165.7) (width 0.2) (layer "B.Cu") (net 13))
 (segment (start 39.181775 167.108174) (end 39.189949 167.1) (width 0.2) (layer "B.Cu") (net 13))
 (segment (start 47.4 166) (end 48.6 166) (width 0.2) (layer "B.Cu") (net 13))
 (segment (start 39.189949 167.1) (end 43 167.1) (width 0.2) (layer "B.Cu") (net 13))
 (segment (start 46.8 165.4) (end 47.4 166) (width 0.2) (layer "B.Cu") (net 13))
 (segment (start 46.7245 164.8) (end 46.8 164.8755) (width 0.2) (layer "B.Cu") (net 13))
 (segment (start 44.450497 172) (end 48.65 172) (width 0.2) (layer "F.Cu") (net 11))
 (segment (start 43.1 170.649503) (end 44.450497 172) (width 0.2) (layer "F.Cu") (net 11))
 (segment (start 37.8 165) (end 37.26 164.46) (width 0.2) (layer "F.Cu") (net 11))
 (segment (start 37.26 164.46) (end 36.525 164.46) (width 0.2) (layer "F.Cu") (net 11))
 (via (at 43.1 170.649503) (size 0.55) (drill 0.3) (layers "F.Cu" "B.Cu") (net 11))
 (via (at 37.8 165) (size 0.55) (drill 0.3) (layers "F.Cu" "B.Cu") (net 11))
 (segment (start 38.374511 166.537971) (end 38.374511 165.574511) (width 0.2) (layer "B.Cu") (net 11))
 (segment (start 38.19952 166.712962) (end 38.374511 166.537971) (width 0.2) (layer "B.Cu") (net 11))
 (segment (start 40.549503 170.649503) (end 38.19952 168.29952) (width 0.2) (layer "B.Cu") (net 11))
 (segment (start 38.374511 165.574511) (end 37.8 165) (width 0.2) (layer "B.Cu") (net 11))
 (segment (start 43.1 170.649503) (end 40.549503 170.649503) (width 0.2) (layer "B.Cu") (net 11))
 (segment (start 38.19952 168.29952) (end 38.19952 166.712962) (width 0.2) (layer "B.Cu") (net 11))
 (segment (start 43.1 169.9) (end 47.3 169.9) (width 0.2) (layer "F.Cu") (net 10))
 (segment (start 36.99 163.19) (end 36.525 163.19) (width 0.2) (layer "F.Cu") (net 10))
 (segment (start 37.8 164) (end 36.99 163.19) (width 0.2) (layer "F.Cu") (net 10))
 (segment (start 37.9 164) (end 37.8 164) (width 0.2) (layer "F.Cu") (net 10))
 (segment (start 47.3 169.9) (end 47.4 170) (width 0.2) (layer "F.Cu") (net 10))
 (via (at 37.9 164) (size 0.55) (drill 0.3) (layers "F.Cu" "B.Cu") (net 10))
 (via (at 43.1 169.9) (size 0.55) (drill 0.3) (layers "F.Cu" "B.Cu") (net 10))
 (segment (start 38.77403 164.87403) (end 38.77403 166.703458) (width 0.2) (layer "B.Cu") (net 10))
 (segment (start 38.77403 166.703458) (end 38.59904 166.878448) (width 0.2) (layer "B.Cu") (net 10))
 (segment (start 40.5 169.9) (end 43.1 169.9) (width 0.2) (layer "B.Cu") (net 10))
 (segment (start 38.59904 167.99904) (end 40.5 169.9) (width 0.2) (layer "B.Cu") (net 10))
 (segment (start 38.59904 166.878448) (end 38.59904 167.99904) (width 0.2) (layer "B.Cu") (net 10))
 (segment (start 37.9 164) (end 38.77403 164.87403) (width 0.2) (layer "B.Cu") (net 10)))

